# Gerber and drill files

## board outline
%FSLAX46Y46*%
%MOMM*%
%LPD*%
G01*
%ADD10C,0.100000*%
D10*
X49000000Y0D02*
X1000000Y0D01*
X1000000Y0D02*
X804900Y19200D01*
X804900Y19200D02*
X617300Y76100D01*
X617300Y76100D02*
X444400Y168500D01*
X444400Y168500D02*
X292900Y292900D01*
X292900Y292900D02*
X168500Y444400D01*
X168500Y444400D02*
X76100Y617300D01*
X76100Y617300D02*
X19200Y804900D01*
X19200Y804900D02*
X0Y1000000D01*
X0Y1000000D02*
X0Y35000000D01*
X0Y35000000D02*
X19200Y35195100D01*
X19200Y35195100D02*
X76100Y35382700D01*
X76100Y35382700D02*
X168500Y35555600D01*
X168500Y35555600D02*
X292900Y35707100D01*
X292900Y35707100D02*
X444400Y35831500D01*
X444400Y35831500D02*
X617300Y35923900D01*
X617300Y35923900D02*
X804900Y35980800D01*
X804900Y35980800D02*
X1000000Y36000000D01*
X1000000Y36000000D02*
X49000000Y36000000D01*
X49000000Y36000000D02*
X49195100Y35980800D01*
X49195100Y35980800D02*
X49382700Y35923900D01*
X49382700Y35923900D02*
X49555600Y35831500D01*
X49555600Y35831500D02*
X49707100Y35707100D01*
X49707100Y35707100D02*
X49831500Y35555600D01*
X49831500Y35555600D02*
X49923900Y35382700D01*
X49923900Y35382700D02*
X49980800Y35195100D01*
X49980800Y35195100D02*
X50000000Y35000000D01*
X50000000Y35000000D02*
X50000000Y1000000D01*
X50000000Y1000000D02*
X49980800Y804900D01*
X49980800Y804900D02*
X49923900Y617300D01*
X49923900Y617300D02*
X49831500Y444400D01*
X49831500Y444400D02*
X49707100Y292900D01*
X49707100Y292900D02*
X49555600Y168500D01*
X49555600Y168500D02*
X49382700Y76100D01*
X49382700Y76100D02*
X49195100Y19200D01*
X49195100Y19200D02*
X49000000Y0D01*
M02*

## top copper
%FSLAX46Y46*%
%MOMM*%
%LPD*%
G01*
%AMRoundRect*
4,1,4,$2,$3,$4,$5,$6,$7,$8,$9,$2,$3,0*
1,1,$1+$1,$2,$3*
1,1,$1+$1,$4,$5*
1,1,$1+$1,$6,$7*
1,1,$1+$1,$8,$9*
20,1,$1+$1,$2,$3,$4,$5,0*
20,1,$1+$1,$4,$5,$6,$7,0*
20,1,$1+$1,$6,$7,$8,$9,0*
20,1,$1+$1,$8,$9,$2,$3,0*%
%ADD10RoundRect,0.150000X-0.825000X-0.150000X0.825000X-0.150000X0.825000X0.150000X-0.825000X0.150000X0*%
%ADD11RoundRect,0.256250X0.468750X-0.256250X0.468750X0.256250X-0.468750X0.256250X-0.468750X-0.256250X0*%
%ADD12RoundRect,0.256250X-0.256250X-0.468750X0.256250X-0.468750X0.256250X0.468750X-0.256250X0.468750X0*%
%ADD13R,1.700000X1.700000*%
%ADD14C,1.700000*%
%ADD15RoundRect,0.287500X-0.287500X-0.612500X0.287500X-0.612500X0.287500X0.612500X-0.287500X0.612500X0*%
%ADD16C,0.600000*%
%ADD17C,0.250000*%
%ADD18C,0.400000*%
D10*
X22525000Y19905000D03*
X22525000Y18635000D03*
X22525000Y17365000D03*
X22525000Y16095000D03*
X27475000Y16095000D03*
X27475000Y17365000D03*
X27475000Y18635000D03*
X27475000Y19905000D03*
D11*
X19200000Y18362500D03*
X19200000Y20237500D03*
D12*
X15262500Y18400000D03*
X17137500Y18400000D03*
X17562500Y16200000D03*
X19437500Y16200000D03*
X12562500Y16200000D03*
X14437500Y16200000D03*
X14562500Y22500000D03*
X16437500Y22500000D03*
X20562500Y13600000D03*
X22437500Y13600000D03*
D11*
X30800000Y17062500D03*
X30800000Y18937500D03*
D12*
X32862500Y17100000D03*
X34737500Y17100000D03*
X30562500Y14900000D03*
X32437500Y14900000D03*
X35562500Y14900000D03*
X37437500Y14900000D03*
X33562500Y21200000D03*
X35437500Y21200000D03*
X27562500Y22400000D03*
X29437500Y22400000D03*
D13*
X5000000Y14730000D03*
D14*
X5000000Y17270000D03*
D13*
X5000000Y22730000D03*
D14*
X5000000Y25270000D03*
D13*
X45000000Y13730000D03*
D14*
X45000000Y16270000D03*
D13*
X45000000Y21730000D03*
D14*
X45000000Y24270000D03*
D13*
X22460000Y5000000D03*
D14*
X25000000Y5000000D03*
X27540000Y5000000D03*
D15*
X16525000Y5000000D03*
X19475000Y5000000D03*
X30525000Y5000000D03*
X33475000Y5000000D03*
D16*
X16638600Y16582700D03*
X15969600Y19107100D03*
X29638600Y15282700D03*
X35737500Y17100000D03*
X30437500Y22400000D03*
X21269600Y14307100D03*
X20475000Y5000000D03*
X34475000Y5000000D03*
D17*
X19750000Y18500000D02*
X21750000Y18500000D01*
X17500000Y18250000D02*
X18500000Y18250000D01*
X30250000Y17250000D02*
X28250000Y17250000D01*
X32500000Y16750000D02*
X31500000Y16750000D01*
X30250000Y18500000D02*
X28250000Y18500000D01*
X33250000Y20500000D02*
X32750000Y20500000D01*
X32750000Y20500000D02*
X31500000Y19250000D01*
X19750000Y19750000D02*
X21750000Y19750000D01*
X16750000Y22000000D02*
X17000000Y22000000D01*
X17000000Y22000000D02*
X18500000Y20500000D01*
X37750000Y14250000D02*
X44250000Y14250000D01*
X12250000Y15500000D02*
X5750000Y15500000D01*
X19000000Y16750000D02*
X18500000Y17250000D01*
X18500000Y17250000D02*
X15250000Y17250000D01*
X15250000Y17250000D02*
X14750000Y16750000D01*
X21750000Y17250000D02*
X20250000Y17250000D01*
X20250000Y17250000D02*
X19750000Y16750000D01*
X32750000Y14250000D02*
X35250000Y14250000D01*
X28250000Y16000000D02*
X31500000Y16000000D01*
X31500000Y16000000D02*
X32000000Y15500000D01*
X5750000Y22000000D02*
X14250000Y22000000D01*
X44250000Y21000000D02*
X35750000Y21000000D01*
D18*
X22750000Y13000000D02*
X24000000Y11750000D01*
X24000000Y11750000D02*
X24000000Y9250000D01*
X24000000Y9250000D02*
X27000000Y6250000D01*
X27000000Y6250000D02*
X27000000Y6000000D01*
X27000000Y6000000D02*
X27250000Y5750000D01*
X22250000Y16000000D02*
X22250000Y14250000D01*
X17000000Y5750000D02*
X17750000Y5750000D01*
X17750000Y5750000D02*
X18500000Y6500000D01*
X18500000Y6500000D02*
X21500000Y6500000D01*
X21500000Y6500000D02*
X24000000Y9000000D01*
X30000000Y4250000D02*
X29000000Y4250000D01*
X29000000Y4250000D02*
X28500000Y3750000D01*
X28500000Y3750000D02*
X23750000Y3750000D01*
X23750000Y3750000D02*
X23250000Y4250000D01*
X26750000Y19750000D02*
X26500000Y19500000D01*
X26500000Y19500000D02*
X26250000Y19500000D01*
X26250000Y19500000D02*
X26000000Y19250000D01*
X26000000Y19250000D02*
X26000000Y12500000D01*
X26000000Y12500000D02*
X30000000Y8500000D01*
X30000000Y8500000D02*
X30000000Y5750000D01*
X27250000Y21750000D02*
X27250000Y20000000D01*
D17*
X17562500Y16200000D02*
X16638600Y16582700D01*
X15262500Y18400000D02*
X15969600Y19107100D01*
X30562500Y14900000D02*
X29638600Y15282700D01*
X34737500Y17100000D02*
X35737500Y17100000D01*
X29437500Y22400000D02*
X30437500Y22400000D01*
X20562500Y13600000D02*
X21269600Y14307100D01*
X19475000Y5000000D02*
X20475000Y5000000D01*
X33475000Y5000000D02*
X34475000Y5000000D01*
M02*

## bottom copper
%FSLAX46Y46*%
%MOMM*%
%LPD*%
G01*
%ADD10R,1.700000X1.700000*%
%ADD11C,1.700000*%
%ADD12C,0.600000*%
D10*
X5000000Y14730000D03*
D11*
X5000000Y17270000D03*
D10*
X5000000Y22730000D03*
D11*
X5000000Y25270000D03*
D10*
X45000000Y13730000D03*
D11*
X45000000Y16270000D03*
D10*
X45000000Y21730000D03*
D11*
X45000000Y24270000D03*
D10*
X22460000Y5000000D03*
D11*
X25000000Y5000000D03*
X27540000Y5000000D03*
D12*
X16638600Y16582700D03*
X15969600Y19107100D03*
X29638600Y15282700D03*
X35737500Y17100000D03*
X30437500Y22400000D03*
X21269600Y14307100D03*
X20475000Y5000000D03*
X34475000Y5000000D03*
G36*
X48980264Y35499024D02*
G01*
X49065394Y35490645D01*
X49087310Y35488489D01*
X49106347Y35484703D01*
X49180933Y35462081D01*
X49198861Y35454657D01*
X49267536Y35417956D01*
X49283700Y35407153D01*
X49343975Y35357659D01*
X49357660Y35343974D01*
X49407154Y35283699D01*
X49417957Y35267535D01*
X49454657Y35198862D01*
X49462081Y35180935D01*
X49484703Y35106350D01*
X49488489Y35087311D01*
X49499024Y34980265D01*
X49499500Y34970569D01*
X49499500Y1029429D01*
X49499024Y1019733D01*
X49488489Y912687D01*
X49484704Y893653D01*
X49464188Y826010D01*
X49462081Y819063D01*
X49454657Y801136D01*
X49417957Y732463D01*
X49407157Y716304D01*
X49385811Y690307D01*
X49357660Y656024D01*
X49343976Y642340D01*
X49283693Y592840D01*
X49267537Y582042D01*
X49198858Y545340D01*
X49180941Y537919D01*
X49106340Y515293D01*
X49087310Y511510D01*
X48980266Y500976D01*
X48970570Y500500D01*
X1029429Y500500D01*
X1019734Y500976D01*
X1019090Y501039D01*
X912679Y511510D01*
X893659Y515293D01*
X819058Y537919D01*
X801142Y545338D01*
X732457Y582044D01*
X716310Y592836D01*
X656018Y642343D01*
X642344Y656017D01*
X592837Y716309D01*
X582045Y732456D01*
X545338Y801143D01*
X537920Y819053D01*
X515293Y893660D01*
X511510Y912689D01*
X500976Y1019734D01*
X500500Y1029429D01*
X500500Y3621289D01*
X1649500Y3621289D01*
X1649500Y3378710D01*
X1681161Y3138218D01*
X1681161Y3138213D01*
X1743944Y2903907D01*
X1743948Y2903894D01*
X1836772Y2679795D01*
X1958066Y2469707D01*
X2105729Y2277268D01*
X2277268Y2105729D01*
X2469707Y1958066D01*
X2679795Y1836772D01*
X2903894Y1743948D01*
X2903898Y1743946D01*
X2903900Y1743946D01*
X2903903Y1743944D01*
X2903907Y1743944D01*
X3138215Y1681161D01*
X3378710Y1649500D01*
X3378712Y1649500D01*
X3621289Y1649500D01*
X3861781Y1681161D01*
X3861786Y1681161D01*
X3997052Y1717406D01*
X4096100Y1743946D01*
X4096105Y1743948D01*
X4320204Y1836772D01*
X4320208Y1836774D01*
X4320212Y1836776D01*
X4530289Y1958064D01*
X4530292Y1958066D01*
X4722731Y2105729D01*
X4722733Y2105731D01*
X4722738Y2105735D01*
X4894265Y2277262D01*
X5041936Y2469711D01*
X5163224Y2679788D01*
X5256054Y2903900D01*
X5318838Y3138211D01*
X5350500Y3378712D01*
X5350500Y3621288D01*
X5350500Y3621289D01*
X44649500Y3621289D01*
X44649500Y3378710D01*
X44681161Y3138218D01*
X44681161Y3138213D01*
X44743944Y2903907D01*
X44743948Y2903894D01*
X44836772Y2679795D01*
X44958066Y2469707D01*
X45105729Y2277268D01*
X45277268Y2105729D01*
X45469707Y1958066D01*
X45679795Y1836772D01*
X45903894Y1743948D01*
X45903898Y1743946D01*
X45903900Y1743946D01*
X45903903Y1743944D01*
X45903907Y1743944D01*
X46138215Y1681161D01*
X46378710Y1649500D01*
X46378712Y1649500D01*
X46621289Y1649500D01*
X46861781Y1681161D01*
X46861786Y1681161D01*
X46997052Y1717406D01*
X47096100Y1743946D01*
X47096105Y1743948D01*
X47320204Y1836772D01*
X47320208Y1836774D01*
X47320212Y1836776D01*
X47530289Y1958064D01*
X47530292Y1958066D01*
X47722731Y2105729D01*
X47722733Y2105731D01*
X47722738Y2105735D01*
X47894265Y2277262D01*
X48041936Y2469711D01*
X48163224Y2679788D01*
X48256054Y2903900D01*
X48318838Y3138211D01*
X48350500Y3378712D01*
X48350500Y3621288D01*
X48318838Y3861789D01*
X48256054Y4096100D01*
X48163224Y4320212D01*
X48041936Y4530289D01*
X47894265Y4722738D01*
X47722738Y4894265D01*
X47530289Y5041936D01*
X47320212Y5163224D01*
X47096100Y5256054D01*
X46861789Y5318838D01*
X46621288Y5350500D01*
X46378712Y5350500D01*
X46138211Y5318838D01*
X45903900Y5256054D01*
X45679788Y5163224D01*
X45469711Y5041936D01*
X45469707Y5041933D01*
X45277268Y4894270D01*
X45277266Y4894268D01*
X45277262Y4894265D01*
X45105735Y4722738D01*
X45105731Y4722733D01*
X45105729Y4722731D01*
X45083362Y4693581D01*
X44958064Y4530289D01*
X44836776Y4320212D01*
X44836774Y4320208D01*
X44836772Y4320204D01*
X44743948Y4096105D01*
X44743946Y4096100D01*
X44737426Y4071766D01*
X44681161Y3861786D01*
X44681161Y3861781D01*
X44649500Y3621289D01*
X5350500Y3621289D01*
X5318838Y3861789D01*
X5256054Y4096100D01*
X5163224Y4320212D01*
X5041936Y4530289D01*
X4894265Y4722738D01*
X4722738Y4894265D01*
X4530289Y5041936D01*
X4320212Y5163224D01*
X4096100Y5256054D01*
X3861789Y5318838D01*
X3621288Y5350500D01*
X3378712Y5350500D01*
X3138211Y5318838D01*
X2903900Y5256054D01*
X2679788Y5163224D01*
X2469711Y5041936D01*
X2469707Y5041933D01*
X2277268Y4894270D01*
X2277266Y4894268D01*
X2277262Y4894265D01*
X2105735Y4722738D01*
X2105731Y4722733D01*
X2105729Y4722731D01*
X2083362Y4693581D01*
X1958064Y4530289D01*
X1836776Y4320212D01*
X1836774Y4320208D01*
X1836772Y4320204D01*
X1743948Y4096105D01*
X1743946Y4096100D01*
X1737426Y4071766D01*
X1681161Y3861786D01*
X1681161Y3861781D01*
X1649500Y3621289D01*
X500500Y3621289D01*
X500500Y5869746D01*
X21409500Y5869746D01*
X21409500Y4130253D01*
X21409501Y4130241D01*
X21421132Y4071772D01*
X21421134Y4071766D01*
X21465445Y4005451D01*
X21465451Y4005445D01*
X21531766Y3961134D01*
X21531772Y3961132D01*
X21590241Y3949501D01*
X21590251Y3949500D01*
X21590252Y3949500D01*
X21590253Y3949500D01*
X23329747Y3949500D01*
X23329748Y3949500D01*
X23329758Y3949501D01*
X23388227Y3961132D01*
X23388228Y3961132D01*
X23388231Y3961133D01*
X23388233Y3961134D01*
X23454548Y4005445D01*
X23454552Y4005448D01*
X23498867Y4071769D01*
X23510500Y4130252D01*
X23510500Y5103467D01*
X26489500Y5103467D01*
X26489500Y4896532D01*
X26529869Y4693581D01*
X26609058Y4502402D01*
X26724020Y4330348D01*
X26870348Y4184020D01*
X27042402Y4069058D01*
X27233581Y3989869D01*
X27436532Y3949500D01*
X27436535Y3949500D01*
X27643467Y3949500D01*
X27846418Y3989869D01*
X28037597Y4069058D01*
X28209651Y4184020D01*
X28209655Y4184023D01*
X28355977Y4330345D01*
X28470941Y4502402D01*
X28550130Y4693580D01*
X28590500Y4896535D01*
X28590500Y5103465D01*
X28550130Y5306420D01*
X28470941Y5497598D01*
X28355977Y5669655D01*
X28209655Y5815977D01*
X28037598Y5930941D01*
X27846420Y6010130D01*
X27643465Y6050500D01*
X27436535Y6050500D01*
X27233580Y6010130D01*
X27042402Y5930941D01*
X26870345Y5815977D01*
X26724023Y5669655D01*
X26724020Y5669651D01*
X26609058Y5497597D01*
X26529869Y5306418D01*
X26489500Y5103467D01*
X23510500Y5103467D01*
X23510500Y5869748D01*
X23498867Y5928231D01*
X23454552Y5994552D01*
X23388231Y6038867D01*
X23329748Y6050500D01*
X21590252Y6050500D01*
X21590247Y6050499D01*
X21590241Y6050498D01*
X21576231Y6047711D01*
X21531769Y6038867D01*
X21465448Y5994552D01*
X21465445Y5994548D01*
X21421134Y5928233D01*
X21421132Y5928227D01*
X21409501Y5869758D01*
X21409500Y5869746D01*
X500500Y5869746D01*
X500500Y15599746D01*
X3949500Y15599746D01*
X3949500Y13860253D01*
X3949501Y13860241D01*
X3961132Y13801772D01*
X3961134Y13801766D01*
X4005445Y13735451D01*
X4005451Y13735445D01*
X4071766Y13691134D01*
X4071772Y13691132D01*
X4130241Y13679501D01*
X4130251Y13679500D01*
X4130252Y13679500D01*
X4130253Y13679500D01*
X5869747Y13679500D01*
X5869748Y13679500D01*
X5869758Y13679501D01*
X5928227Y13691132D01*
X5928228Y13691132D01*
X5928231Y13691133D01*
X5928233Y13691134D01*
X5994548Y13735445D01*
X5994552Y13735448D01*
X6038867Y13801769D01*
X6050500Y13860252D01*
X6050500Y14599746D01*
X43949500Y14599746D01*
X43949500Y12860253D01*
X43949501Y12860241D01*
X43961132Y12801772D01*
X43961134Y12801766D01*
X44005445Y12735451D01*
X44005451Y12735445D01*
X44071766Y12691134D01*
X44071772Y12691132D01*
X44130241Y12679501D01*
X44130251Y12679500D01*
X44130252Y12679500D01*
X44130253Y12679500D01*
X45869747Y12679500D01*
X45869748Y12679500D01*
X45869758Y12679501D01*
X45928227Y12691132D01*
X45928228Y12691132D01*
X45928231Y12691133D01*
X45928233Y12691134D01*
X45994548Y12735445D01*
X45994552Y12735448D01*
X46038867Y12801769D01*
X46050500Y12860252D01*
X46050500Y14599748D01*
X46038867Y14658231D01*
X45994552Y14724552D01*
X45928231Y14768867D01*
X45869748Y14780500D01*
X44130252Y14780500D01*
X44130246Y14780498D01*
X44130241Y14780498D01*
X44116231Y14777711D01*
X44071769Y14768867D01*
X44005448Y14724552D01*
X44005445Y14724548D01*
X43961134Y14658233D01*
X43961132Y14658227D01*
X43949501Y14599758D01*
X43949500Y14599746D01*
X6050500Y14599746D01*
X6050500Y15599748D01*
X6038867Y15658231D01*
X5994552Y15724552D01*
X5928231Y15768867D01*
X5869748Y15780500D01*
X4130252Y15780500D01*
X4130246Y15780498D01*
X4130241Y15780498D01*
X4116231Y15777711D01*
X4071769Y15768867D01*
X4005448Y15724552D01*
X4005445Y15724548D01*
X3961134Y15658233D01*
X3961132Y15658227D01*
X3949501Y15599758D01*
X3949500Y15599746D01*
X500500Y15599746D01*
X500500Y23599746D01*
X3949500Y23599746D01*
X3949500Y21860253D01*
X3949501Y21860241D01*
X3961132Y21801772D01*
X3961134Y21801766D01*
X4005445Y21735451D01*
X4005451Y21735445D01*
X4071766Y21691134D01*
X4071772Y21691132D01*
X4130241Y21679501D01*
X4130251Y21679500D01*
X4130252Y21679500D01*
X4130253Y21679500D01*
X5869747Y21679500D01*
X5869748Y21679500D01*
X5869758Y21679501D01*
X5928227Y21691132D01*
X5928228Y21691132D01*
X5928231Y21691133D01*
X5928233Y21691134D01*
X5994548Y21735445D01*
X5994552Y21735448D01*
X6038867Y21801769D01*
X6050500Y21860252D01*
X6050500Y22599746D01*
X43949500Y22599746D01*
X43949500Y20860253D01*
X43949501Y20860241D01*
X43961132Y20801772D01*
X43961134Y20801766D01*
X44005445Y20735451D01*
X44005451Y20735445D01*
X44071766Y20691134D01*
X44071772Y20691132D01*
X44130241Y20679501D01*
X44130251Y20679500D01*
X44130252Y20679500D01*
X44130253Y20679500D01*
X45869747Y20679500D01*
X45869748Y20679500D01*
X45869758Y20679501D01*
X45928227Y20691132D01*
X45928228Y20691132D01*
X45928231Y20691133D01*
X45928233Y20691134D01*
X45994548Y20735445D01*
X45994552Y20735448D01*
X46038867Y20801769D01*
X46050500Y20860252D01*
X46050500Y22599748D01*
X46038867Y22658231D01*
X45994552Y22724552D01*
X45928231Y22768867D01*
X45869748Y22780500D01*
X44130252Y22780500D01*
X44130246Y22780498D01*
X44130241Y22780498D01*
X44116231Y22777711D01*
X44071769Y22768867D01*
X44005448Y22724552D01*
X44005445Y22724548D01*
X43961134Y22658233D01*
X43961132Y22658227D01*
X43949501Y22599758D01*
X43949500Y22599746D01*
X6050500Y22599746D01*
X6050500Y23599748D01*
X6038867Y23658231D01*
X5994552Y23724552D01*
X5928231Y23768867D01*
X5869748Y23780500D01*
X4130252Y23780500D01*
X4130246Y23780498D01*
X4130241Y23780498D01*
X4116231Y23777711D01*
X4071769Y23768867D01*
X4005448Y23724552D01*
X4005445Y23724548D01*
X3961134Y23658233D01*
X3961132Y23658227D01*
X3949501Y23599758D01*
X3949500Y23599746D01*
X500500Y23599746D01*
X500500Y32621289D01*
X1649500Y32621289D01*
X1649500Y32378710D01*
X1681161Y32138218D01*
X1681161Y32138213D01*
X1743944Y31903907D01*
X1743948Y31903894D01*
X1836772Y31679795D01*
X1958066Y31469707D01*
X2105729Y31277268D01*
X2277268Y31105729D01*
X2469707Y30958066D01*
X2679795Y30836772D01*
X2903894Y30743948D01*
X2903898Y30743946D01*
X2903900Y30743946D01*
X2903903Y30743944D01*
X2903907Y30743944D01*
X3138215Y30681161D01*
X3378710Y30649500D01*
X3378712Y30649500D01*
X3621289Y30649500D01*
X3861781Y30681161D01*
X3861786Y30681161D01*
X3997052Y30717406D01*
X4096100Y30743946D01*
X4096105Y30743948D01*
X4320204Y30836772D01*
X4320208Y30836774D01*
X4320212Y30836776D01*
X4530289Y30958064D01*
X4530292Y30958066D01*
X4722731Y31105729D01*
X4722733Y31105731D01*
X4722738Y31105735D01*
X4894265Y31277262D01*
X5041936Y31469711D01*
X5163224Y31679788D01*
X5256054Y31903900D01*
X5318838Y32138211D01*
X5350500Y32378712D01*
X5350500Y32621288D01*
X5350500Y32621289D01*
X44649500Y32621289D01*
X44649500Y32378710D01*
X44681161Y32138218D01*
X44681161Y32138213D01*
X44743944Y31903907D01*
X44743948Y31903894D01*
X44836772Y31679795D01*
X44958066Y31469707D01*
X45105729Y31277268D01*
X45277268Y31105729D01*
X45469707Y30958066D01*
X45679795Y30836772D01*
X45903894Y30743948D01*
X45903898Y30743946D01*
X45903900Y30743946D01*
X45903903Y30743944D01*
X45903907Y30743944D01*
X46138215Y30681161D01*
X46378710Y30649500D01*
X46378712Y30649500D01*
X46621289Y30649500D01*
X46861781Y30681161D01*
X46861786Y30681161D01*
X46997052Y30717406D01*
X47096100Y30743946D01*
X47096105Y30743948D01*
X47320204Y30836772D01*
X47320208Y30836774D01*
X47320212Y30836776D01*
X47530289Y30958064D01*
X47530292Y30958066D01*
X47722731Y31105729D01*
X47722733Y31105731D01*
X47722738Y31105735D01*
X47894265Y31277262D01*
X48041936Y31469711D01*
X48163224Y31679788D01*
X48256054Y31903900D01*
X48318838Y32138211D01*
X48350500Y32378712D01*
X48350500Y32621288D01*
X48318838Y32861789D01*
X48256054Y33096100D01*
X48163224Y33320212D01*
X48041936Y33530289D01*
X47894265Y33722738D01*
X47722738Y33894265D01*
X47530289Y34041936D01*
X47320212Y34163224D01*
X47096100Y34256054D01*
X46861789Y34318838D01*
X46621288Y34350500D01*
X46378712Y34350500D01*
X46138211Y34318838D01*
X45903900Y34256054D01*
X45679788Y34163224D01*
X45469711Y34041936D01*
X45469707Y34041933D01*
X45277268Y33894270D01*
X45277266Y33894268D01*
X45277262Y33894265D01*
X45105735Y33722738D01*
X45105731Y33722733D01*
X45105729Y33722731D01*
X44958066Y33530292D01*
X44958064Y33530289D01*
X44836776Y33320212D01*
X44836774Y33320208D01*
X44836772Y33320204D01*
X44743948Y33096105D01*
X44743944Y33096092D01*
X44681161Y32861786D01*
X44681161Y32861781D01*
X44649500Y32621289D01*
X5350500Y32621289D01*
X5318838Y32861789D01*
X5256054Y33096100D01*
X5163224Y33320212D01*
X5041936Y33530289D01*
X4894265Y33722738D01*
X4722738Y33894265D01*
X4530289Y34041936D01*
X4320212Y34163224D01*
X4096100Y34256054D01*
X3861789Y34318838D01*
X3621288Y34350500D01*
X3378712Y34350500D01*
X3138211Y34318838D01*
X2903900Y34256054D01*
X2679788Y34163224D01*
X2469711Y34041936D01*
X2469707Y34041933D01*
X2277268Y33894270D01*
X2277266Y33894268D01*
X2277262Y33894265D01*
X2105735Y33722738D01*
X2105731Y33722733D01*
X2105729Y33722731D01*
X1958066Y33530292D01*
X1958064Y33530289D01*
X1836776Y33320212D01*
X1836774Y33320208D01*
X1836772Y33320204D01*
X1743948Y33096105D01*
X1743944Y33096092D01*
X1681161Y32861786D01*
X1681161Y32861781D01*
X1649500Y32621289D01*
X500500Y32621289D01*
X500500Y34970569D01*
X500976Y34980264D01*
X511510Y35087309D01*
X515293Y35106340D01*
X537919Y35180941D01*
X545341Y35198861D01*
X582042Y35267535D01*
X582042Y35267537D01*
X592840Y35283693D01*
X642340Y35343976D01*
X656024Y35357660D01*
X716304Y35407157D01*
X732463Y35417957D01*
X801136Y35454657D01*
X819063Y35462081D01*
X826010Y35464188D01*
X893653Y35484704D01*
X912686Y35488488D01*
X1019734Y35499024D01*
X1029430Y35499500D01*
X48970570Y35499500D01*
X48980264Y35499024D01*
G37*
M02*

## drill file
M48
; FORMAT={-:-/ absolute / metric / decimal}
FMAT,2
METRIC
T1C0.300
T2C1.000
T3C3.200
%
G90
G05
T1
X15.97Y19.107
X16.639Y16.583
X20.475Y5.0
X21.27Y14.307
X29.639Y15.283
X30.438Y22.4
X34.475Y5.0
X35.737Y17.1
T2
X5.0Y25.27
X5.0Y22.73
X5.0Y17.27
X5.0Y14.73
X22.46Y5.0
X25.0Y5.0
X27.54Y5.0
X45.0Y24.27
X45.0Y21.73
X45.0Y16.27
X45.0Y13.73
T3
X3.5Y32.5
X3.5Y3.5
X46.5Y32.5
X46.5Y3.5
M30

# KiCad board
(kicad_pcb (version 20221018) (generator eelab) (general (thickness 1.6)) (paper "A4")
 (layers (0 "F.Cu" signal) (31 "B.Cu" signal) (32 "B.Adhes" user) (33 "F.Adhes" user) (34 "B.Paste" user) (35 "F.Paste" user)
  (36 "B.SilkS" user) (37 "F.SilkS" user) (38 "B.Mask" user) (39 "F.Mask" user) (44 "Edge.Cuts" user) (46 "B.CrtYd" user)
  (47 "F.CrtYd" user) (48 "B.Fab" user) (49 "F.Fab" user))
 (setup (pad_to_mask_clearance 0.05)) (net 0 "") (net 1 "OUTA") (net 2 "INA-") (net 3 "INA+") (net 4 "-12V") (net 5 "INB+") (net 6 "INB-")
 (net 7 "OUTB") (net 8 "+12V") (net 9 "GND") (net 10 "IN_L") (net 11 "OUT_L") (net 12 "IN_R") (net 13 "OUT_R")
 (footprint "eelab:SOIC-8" (layer "F.Cu") (at 25.0000 -18.0000 0)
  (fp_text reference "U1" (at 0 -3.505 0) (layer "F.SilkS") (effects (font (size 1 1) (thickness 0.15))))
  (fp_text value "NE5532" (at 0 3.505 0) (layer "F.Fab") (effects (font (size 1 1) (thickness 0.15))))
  (pad "1" smd roundrect (at -2.4750 -1.9050 0) (size 1.9500 0.6000) (layers "F.Cu" "F.Paste" "F.Mask") (roundrect_rratio 0.25)
   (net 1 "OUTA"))
  (pad "2" smd roundrect (at -2.4750 -0.6350 0) (size 1.9500 0.6000) (layers "F.Cu" "F.Paste" "F.Mask") (roundrect_rratio 0.25)
   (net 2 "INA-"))
  (pad "3" smd roundrect (at -2.4750 0.6350 0) (size 1.9500 0.6000) (layers "F.Cu" "F.Paste" "F.Mask") (roundrect_rratio 0.25)
   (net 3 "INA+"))
  (pad "4" smd roundrect (at -2.4750 1.9050 0) (size 1.9500 0.6000) (layers "F.Cu" "F.Paste" "F.Mask") (roundrect_rratio 0.25)
   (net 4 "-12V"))
  (pad "5" smd roundrect (at 2.4750 1.9050 0) (size 1.9500 0.6000) (layers "F.Cu" "F.Paste" "F.Mask") (roundrect_rratio 0.25) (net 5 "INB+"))
  (pad "6" smd roundrect (at 2.4750 0.6350 0) (size 1.9500 0.6000) (layers "F.Cu" "F.Paste" "F.Mask") (roundrect_rratio 0.25) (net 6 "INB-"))
  (pad "7" smd roundrect (at 2.4750 -0.6350 0) (size 1.9500 0.6000) (layers "F.Cu" "F.Paste" "F.Mask") (roundrect_rratio 0.25)
   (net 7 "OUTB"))
  (pad "8" smd roundrect (at 2.4750 -1.9050 0) (size 1.9500 0.6000) (layers "F.Cu" "F.Paste" "F.Mask") (roundrect_rratio 0.25)
   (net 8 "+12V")))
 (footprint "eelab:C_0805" (layer "F.Cu") (at 19.2000 -19.3000 90)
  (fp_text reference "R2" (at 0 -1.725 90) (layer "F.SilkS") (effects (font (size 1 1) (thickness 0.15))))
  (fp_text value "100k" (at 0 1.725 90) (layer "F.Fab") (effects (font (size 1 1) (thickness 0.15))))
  (pad "1" smd roundrect (at -0.9375 0.0000 90) (size 1.0250 1.4500) (layers "F.Cu" "F.Paste" "F.Mask") (roundrect_rratio 0.25)
   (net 2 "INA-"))
  (pad "2" smd roundrect (at 0.9375 0.0000 90) (size 1.0250 1.4500) (layers "F.Cu" "F.Paste" "F.Mask") (roundrect_rratio 0.25)
   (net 1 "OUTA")))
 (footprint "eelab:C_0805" (layer "F.Cu") (at 16.2000 -18.4000 0)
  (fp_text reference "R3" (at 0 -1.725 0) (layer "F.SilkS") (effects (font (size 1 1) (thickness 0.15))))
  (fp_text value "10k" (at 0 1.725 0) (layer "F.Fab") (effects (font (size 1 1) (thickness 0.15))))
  (pad "1" smd roundrect (at -0.9375 0.0000 0) (size 1.0250 1.4500) (layers "F.Cu" "F.Paste" "F.Mask") (roundrect_rratio 0.25) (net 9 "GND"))
  (pad "2" smd roundrect (at 0.9375 0.0000 0) (size 1.0250 1.4500) (layers "F.Cu" "F.Paste" "F.Mask") (roundrect_rratio 0.25) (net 2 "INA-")))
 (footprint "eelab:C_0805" (layer "F.Cu") (at 18.5000 -16.2000 0)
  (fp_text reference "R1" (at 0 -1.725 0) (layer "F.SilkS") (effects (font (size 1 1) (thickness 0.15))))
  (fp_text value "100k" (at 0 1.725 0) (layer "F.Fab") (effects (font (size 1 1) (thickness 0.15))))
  (pad "1" smd roundrect (at -0.9375 0.0000 0) (size 1.0250 1.4500) (layers "F.Cu" "F.Paste" "F.Mask") (roundrect_rratio 0.25) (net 9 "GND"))
  (pad "2" smd roundrect (at 0.9375 0.0000 0) (size 1.0250 1.4500) (layers "F.Cu" "F.Paste" "F.Mask") (roundrect_rratio 0.25) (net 3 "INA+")))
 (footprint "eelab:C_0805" (layer "F.Cu") (at 13.5000 -16.2000 0)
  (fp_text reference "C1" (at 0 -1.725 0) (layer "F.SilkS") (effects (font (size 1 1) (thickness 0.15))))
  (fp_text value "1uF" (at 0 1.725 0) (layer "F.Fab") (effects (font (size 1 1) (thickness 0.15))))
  (pad "1" smd roundrect (at -0.9375 0.0000 0) (size 1.0250 1.4500) (layers "F.Cu" "F.Paste" "F.Mask") (roundrect_rratio 0.25)
   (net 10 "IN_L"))
  (pad "2" smd roundrect (at 0.9375 0.0000 0) (size 1.0250 1.4500) (layers "F.Cu" "F.Paste" "F.Mask") (roundrect_rratio 0.25) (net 3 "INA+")))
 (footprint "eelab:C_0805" (layer "F.Cu") (at 15.5000 -22.5000 0)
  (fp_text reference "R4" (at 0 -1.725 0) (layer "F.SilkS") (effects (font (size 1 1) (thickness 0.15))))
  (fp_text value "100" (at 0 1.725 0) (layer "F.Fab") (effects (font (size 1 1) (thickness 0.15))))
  (pad "1" smd roundrect (at -0.9375 0.0000 0) (size 1.0250 1.4500) (layers "F.Cu" "F.Paste" "F.Mask") (roundrect_rratio 0.25)
   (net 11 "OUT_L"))
  (pad "2" smd roundrect (at 0.9375 0.0000 0) (size 1.0250 1.4500) (layers "F.Cu" "F.Paste" "F.Mask") (roundrect_rratio 0.25) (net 1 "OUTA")))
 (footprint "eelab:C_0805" (layer "F.Cu") (at 21.5000 -13.6000 0)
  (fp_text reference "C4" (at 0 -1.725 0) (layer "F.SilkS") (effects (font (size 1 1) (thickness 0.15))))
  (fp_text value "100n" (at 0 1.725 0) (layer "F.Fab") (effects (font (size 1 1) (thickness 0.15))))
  (pad "1" smd roundrect (at -0.9375 0.0000 0) (size 1.0250 1.4500) (layers "F.Cu" "F.Paste" "F.Mask") (roundrect_rratio 0.25) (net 9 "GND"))
  (pad "2" smd roundrect (at 0.9375 0.0000 0) (size 1.0250 1.4500) (layers "F.Cu" "F.Paste" "F.Mask") (roundrect_rratio 0.25) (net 4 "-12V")))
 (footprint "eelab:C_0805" (layer "F.Cu") (at 30.8000 -18.0000 90)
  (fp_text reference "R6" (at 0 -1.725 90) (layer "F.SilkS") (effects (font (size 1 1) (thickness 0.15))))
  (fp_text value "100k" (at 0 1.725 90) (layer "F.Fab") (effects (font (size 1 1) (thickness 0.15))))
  (pad "1" smd roundrect (at -0.9375 0.0000 90) (size 1.0250 1.4500) (layers "F.Cu" "F.Paste" "F.Mask") (roundrect_rratio 0.25)
   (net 6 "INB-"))
  (pad "2" smd roundrect (at 0.9375 0.0000 90) (size 1.0250 1.4500) (layers "F.Cu" "F.Paste" "F.Mask") (roundrect_rratio 0.25)
   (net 7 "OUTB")))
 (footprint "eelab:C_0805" (layer "F.Cu") (at 33.8000 -17.1000 0)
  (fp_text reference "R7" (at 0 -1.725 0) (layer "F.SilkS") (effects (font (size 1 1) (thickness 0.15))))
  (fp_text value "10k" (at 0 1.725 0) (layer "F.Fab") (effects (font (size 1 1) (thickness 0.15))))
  (pad "1" smd roundrect (at -0.9375 0.0000 0) (size 1.0250 1.4500) (layers "F.Cu" "F.Paste" "F.Mask") (roundrect_rratio 0.25)
   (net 6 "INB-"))
  (pad "2" smd roundrect (at 0.9375 0.0000 0) (size 1.0250 1.4500) (layers "F.Cu" "F.Paste" "F.Mask") (roundrect_rratio 0.25) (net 9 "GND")))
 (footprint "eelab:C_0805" (layer "F.Cu") (at 31.5000 -14.9000 0)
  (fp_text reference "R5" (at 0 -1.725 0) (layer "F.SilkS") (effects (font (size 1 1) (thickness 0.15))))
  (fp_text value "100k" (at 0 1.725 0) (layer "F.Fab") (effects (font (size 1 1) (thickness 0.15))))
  (pad "1" smd roundrect (at -0.9375 0.0000 0) (size 1.0250 1.4500) (layers "F.Cu" "F.Paste" "F.Mask") (roundrect_rratio 0.25) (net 9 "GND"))
  (pad "2" smd roundrect (at 0.9375 0.0000 0) (size 1.0250 1.4500) (layers "F.Cu" "F.Paste" "F.Mask") (roundrect_rratio 0.25) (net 5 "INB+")))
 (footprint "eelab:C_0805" (layer "F.Cu") (at 36.5000 -14.9000 0)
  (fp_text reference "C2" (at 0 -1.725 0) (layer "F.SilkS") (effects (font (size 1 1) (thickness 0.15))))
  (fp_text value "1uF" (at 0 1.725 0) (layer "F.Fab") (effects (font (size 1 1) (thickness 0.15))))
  (pad "1" smd roundrect (at -0.9375 0.0000 0) (size 1.0250 1.4500) (layers "F.Cu" "F.Paste" "F.Mask") (roundrect_rratio 0.25)
   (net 5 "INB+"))
  (pad "2" smd roundrect (at 0.9375 0.0000 0) (size 1.0250 1.4500) (layers "F.Cu" "F.Paste" "F.Mask") (roundrect_rratio 0.25)
   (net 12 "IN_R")))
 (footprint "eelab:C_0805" (layer "F.Cu") (at 34.5000 -21.2000 0)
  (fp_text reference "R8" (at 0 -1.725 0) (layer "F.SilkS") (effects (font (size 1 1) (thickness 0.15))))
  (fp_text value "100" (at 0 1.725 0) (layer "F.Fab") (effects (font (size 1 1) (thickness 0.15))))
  (pad "1" smd roundrect (at -0.9375 0.0000 0) (size 1.0250 1.4500) (layers "F.Cu" "F.Paste" "F.Mask") (roundrect_rratio 0.25)
   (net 7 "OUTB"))
  (pad "2" smd roundrect (at 0.9375 0.0000 0) (size 1.0250 1.4500) (layers "F.Cu" "F.Paste" "F.Mask") (roundrect_rratio 0.25)
   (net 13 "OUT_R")))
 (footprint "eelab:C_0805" (layer "F.Cu") (at 28.5000 -22.4000 0)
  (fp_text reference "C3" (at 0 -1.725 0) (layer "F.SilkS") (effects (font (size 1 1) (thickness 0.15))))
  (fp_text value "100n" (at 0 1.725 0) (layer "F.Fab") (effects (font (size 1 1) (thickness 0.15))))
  (pad "1" smd roundrect (at -0.9375 0.0000 0) (size 1.0250 1.4500) (layers "F.Cu" "F.Paste" "F.Mask") (roundrect_rratio 0.25)
   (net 8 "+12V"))
  (pad "2" smd roundrect (at 0.9375 0.0000 0) (size 1.0250 1.4500) (layers "F.Cu" "F.Paste" "F.Mask") (roundrect_rratio 0.25) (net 9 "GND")))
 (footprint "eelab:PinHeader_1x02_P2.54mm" (layer "F.Cu") (at 5.0000 -16.0000 90)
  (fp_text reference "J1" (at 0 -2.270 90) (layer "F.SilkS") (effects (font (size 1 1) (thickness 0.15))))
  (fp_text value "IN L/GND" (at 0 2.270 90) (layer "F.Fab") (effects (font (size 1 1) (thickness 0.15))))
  (pad "1" thru_hole rect (at -1.2700 -0.0000 90) (size 1.7000 1.7000) (drill 1.0) (layers "*.Cu" "*.Mask") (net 10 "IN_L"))
  (pad "2" thru_hole circle (at 1.2700 -0.0000 90) (size 1.7000 1.7000) (drill 1.0) (layers "*.Cu" "*.Mask") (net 9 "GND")))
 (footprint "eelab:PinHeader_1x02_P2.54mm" (layer "F.Cu") (at 5.0000 -24.0000 90)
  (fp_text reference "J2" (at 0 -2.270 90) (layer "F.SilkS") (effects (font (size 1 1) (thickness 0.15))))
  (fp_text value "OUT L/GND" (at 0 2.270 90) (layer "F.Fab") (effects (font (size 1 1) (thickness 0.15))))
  (pad "1" thru_hole rect (at -1.2700 -0.0000 90) (size 1.7000 1.7000) (drill 1.0) (layers "*.Cu" "*.Mask") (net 11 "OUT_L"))
  (pad "2" thru_hole circle (at 1.2700 -0.0000 90) (size 1.7000 1.7000) (drill 1.0) (layers "*.Cu" "*.Mask") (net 9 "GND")))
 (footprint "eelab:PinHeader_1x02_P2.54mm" (layer "F.Cu") (at 45.0000 -15.0000 90)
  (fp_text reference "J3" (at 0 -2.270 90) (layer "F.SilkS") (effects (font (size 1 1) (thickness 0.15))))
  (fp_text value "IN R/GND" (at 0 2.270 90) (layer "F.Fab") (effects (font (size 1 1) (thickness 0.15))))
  (pad "1" thru_hole rect (at -1.2700 -0.0000 90) (size 1.7000 1.7000) (drill 1.0) (layers "*.Cu" "*.Mask") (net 12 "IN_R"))
  (pad "2" thru_hole circle (at 1.2700 -0.0000 90) (size 1.7000 1.7000) (drill 1.0) (layers "*.Cu" "*.Mask") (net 9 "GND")))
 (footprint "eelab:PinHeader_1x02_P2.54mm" (layer "F.Cu") (at 45.0000 -23.0000 90)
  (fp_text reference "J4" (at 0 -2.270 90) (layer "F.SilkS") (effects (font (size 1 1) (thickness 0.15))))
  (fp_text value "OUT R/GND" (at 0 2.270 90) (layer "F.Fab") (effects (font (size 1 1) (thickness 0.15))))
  (pad "1" thru_hole rect (at -1.2700 -0.0000 90) (size 1.7000 1.7000) (drill 1.0) (layers "*.Cu" "*.Mask") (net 13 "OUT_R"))
  (pad "2" thru_hole circle (at 1.2700 -0.0000 90) (size 1.7000 1.7000) (drill 1.0) (layers "*.Cu" "*.Mask") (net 9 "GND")))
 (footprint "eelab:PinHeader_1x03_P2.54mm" (layer "F.Cu") (at 25.0000 -5.0000 0)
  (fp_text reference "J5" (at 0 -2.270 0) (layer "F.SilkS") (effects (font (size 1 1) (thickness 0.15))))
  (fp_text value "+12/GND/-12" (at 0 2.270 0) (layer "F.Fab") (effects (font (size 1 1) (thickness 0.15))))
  (pad "1" thru_hole rect (at -2.5400 -0.0000 0) (size 1.7000 1.7000) (drill 1.0) (layers "*.Cu" "*.Mask") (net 8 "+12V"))
  (pad "2" thru_hole circle (at 0.0000 -0.0000 0) (size 1.7000 1.7000) (drill 1.0) (layers "*.Cu" "*.Mask") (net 9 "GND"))
  (pad "3" thru_hole circle (at 2.5400 -0.0000 0) (size 1.7000 1.7000) (drill 1.0) (layers "*.Cu" "*.Mask") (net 4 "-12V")))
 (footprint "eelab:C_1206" (layer "F.Cu") (at 18.0000 -5.0000 0)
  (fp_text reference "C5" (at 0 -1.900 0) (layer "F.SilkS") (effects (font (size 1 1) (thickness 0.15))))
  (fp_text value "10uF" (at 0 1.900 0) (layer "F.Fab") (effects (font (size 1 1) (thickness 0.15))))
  (pad "1" smd roundrect (at -1.4750 0.0000 0) (size 1.1500 1.8000) (layers "F.Cu" "F.Paste" "F.Mask") (roundrect_rratio 0.25)
   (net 4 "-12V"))
  (pad "2" smd roundrect (at 1.4750 0.0000 0) (size 1.1500 1.8000) (layers "F.Cu" "F.Paste" "F.Mask") (roundrect_rratio 0.25) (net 9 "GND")))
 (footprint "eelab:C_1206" (layer "F.Cu") (at 32.0000 -5.0000 0)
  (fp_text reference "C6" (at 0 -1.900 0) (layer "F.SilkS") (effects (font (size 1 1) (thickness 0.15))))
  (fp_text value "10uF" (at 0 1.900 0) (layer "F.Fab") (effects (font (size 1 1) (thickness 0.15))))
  (pad "1" smd roundrect (at -1.4750 0.0000 0) (size 1.1500 1.8000) (layers "F.Cu" "F.Paste" "F.Mask") (roundrect_rratio 0.25)
   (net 8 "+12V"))
  (pad "2" smd roundrect (at 1.4750 0.0000 0) (size 1.1500 1.8000) (layers "F.Cu" "F.Paste" "F.Mask") (roundrect_rratio 0.25) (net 9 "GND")))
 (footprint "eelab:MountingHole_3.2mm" (layer "F.Cu") (at 3.5000 -3.5000 0)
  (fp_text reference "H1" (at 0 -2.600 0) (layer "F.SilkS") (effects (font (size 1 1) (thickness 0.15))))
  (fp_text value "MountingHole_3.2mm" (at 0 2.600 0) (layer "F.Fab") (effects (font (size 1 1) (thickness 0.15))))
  (pad "" np_thru_hole circle (at 0.0000 0.0000 0) (size 3.2000 3.2000) (drill 3.2) (layers "*.Cu" "*.Mask")))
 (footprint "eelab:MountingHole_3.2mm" (layer "F.Cu") (at 46.5000 -3.5000 0)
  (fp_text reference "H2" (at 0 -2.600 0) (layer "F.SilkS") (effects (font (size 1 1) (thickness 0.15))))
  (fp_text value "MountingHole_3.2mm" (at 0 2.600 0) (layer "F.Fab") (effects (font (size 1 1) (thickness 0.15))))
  (pad "" np_thru_hole circle (at 0.0000 0.0000 0) (size 3.2000 3.2000) (drill 3.2) (layers "*.Cu" "*.Mask")))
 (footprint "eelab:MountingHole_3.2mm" (layer "F.Cu") (at 3.5000 -32.5000 0)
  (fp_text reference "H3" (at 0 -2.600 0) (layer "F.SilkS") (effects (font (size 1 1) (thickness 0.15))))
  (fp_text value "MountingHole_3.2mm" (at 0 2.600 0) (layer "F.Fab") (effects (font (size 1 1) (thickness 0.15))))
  (pad "" np_thru_hole circle (at 0.0000 0.0000 0) (size 3.2000 3.2000) (drill 3.2) (layers "*.Cu" "*.Mask")))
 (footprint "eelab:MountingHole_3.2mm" (layer "F.Cu") (at 46.5000 -32.5000 0)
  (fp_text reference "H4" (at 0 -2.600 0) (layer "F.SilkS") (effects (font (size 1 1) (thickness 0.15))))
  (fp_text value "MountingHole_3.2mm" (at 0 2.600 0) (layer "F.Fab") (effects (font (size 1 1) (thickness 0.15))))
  (pad "" np_thru_hole circle (at 0.0000 0.0000 0) (size 3.2000 3.2000) (drill 3.2) (layers "*.Cu" "*.Mask")))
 (gr_line (start 49.0000 -0.0000) (end 1.0000 -0.0000) (stroke (width 0.1) (type solid)) (layer "Edge.Cuts"))
 (gr_line (start 1.0000 -0.0000) (end 0.8049 -0.0192) (stroke (width 0.1) (type solid)) (layer "Edge.Cuts"))
 (gr_line (start 0.8049 -0.0192) (end 0.6173 -0.0761) (stroke (width 0.1) (type solid)) (layer "Edge.Cuts"))
 (gr_line (start 0.6173 -0.0761) (end 0.4444 -0.1685) (stroke (width 0.1) (type solid)) (layer "Edge.Cuts"))
 (gr_line (start 0.4444 -0.1685) (end 0.2929 -0.2929) (stroke (width 0.1) (type solid)) (layer "Edge.Cuts"))
 (gr_line (start 0.2929 -0.2929) (end 0.1685 -0.4444) (stroke (width 0.1) (type solid)) (layer "Edge.Cuts"))
 (gr_line (start 0.1685 -0.4444) (end 0.0761 -0.6173) (stroke (width 0.1) (type solid)) (layer "Edge.Cuts"))
 (gr_line (start 0.0761 -0.6173) (end 0.0192 -0.8049) (stroke (width 0.1) (type solid)) (layer "Edge.Cuts"))
 (gr_line (start 0.0192 -0.8049) (end 0.0000 -1.0000) (stroke (width 0.1) (type solid)) (layer "Edge.Cuts"))
 (gr_line (start 0.0000 -1.0000) (end 0.0000 -35.0000) (stroke (width 0.1) (type solid)) (layer "Edge.Cuts"))
 (gr_line (start 0.0000 -35.0000) (end 0.0192 -35.1951) (stroke (width 0.1) (type solid)) (layer "Edge.Cuts"))
 (gr_line (start 0.0192 -35.1951) (end 0.0761 -35.3827) (stroke (width 0.1) (type solid)) (layer "Edge.Cuts"))
 (gr_line (start 0.0761 -35.3827) (end 0.1685 -35.5556) (stroke (width 0.1) (type solid)) (layer "Edge.Cuts"))
 (gr_line (start 0.1685 -35.5556) (end 0.2929 -35.7071) (stroke (width 0.1) (type solid)) (layer "Edge.Cuts"))
 (gr_line (start 0.2929 -35.7071) (end 0.4444 -35.8315) (stroke (width 0.1) (type solid)) (layer "Edge.Cuts"))
 (gr_line (start 0.4444 -35.8315) (end 0.6173 -35.9239) (stroke (width 0.1) (type solid)) (layer "Edge.Cuts"))
 (gr_line (start 0.6173 -35.9239) (end 0.8049 -35.9808) (stroke (width 0.1) (type solid)) (layer "Edge.Cuts"))
 (gr_line (start 0.8049 -35.9808) (end 1.0000 -36.0000) (stroke (width 0.1) (type solid)) (layer "Edge.Cuts"))
 (gr_line (start 1.0000 -36.0000) (end 49.0000 -36.0000) (stroke (width 0.1) (type solid)) (layer "Edge.Cuts"))
 (gr_line (start 49.0000 -36.0000) (end 49.1951 -35.9808) (stroke (width 0.1) (type solid)) (layer "Edge.Cuts"))
 (gr_line (start 49.1951 -35.9808) (end 49.3827 -35.9239) (stroke (width 0.1) (type solid)) (layer "Edge.Cuts"))
 (gr_line (start 49.3827 -35.9239) (end 49.5556 -35.8315) (stroke (width 0.1) (type solid)) (layer "Edge.Cuts"))
 (gr_line (start 49.5556 -35.8315) (end 49.7071 -35.7071) (stroke (width 0.1) (type solid)) (layer "Edge.Cuts"))
 (gr_line (start 49.7071 -35.7071) (end 49.8315 -35.5556) (stroke (width 0.1) (type solid)) (layer "Edge.Cuts"))
 (gr_line (start 49.8315 -35.5556) (end 49.9239 -35.3827) (stroke (width 0.1) (type solid)) (layer "Edge.Cuts"))
 (gr_line (start 49.9239 -35.3827) (end 49.9808 -35.1951) (stroke (width 0.1) (type solid)) (layer "Edge.Cuts"))
 (gr_line (start 49.9808 -35.1951) (end 50.0000 -35.0000) (stroke (width 0.1) (type solid)) (layer "Edge.Cuts"))
 (gr_line (start 50.0000 -35.0000) (end 50.0000 -1.0000) (stroke (width 0.1) (type solid)) (layer "Edge.Cuts"))
 (gr_line (start 50.0000 -1.0000) (end 49.9808 -0.8049) (stroke (width 0.1) (type solid)) (layer "Edge.Cuts"))
 (gr_line (start 49.9808 -0.8049) (end 49.9239 -0.6173) (stroke (width 0.1) (type solid)) (layer "Edge.Cuts"))
 (gr_line (start 49.9239 -0.6173) (end 49.8315 -0.4444) (stroke (width 0.1) (type solid)) (layer "Edge.Cuts"))
 (gr_line (start 49.8315 -0.4444) (end 49.7071 -0.2929) (stroke (width 0.1) (type solid)) (layer "Edge.Cuts"))
 (gr_line (start 49.7071 -0.2929) (end 49.5556 -0.1685) (stroke (width 0.1) (type solid)) (layer "Edge.Cuts"))
 (gr_line (start 49.5556 -0.1685) (end 49.3827 -0.0761) (stroke (width 0.1) (type solid)) (layer "Edge.Cuts"))
 (gr_line (start 49.3827 -0.0761) (end 49.1951 -0.0192) (stroke (width 0.1) (type solid)) (layer "Edge.Cuts"))
 (gr_line (start 49.1951 -0.0192) (end 49.0000 -0.0000) (stroke (width 0.1) (type solid)) (layer "Edge.Cuts"))
 (segment (start 19.7500 -18.5000) (end 21.7500 -18.5000) (width 0.25) (layer "F.Cu") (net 2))
 (segment (start 17.5000 -18.2500) (end 18.5000 -18.2500) (width 0.25) (layer "F.Cu") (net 2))
 (segment (start 30.2500 -17.2500) (end 28.2500 -17.2500) (width 0.25) (layer "F.Cu") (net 6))
 (segment (start 32.5000 -16.7500) (end 31.5000 -16.7500) (width 0.25) (layer "F.Cu") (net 6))
 (segment (start 30.2500 -18.5000) (end 28.2500 -18.5000) (width 0.25) (layer "F.Cu") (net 7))
 (segment (start 33.2500 -20.5000) (end 32.7500 -20.5000) (width 0.25) (layer "F.Cu") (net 7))
 (segment (start 32.7500 -20.5000) (end 31.5000 -19.2500) (width 0.25) (layer "F.Cu") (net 7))
 (segment (start 19.7500 -19.7500) (end 21.7500 -19.7500) (width 0.25) (layer "F.Cu") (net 1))
 (segment (start 16.7500 -22.0000) (end 17.0000 -22.0000) (width 0.25) (layer "F.Cu") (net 1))
 (segment (start 17.0000 -22.0000) (end 18.5000 -20.5000) (width 0.25) (layer "F.Cu") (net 1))
 (segment (start 37.7500 -14.2500) (end 44.2500 -14.2500) (width 0.25) (layer "F.Cu") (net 12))
 (segment (start 12.2500 -15.5000) (end 5.7500 -15.5000) (width 0.25) (layer "F.Cu") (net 10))
 (segment (start 19.0000 -16.7500) (end 18.5000 -17.2500) (width 0.25) (layer "F.Cu") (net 3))
 (segment (start 18.5000 -17.2500) (end 15.2500 -17.2500) (width 0.25) (layer "F.Cu") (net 3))
 (segment (start 15.2500 -17.2500) (end 14.7500 -16.7500) (width 0.25) (layer "F.Cu") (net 3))
 (segment (start 21.7500 -17.2500) (end 20.2500 -17.2500) (width 0.25) (layer "F.Cu") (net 3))
 (segment (start 20.2500 -17.2500) (end 19.7500 -16.7500) (width 0.25) (layer "F.Cu") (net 3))
 (segment (start 32.7500 -14.2500) (end 35.2500 -14.2500) (width 0.25) (layer "F.Cu") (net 5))
 (segment (start 28.2500 -16.0000) (end 31.5000 -16.0000) (width 0.25) (layer "F.Cu") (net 5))
 (segment (start 31.5000 -16.0000) (end 32.0000 -15.5000) (width 0.25) (layer "F.Cu") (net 5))
 (segment (start 5.7500 -22.0000) (end 14.2500 -22.0000) (width 0.25) (layer "F.Cu") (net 11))
 (segment (start 44.2500 -21.0000) (end 35.7500 -21.0000) (width 0.25) (layer "F.Cu") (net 13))
 (segment (start 22.7500 -13.0000) (end 24.0000 -11.7500) (width 0.4) (layer "F.Cu") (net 4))
 (segment (start 24.0000 -11.7500) (end 24.0000 -9.2500) (width 0.4) (layer "F.Cu") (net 4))
 (segment (start 24.0000 -9.2500) (end 27.0000 -6.2500) (width 0.4) (layer "F.Cu") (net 4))
 (segment (start 27.0000 -6.2500) (end 27.0000 -6.0000) (width 0.4) (layer "F.Cu") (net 4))
 (segment (start 27.0000 -6.0000) (end 27.2500 -5.7500) (width 0.4) (layer "F.Cu") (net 4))
 (segment (start 22.2500 -16.0000) (end 22.2500 -14.2500) (width 0.4) (layer "F.Cu") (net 4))
 (segment (start 17.0000 -5.7500) (end 17.7500 -5.7500) (width 0.4) (layer "F.Cu") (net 4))
 (segment (start 17.7500 -5.7500) (end 18.5000 -6.5000) (width 0.4) (layer "F.Cu") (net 4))
 (segment (start 18.5000 -6.5000) (end 21.5000 -6.5000) (width 0.4) (layer "F.Cu") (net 4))
 (segment (start 21.5000 -6.5000) (end 24.0000 -9.0000) (width 0.4) (layer "F.Cu") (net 4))
 (segment (start 30.0000 -4.2500) (end 29.0000 -4.2500) (width 0.4) (layer "F.Cu") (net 8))
 (segment (start 29.0000 -4.2500) (end 28.5000 -3.7500) (width 0.4) (layer "F.Cu") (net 8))
 (segment (start 28.5000 -3.7500) (end 23.7500 -3.7500) (width 0.4) (layer "F.Cu") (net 8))
 (segment (start 23.7500 -3.7500) (end 23.2500 -4.2500) (width 0.4) (layer "F.Cu") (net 8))
 (segment (start 26.7500 -19.7500) (end 26.5000 -19.5000) (width 0.4) (layer "F.Cu") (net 8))
 (segment (start 26.5000 -19.5000) (end 26.2500 -19.5000) (width 0.4) (layer "F.Cu") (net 8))
 (segment (start 26.2500 -19.5000) (end 26.0000 -19.2500) (width 0.4) (layer "F.Cu") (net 8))
 (segment (start 26.0000 -19.2500) (end 26.0000 -12.5000) (width 0.4) (layer "F.Cu") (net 8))
 (segment (start 26.0000 -12.5000) (end 30.0000 -8.5000) (width 0.4) (layer "F.Cu") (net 8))
 (segment (start 30.0000 -8.5000) (end 30.0000 -5.7500) (width 0.4) (layer "F.Cu") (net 8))
 (segment (start 27.2500 -21.7500) (end 27.2500 -20.0000) (width 0.4) (layer "F.Cu") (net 8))
 (segment (start 17.5625 -16.2000) (end 16.6386 -16.5827) (width 0.25) (layer "F.Cu") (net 9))
 (segment (start 15.2625 -18.4000) (end 15.9696 -19.1071) (width 0.25) (layer "F.Cu") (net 9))
 (segment (start 30.5625 -14.9000) (end 29.6386 -15.2827) (width 0.25) (layer "F.Cu") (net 9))
 (segment (start 34.7375 -17.1000) (end 35.7375 -17.1000) (width 0.25) (layer "F.Cu") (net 9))
 (segment (start 29.4375 -22.4000) (end 30.4375 -22.4000) (width 0.25) (layer "F.Cu") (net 9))
 (segment (start 20.5625 -13.6000) (end 21.2696 -14.3071) (width 0.25) (layer "F.Cu") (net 9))
 (segment (start 19.4750 -5.0000) (end 20.4750 -5.0000) (width 0.25) (layer "F.Cu") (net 9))
 (segment (start 33.4750 -5.0000) (end 34.4750 -5.0000) (width 0.25) (layer "F.Cu") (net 9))
 (via (at 16.6386 -16.5827) (size 0.6) (drill 0.3) (layers "F.Cu" "B.Cu") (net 9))
 (via (at 15.9696 -19.1071) (size 0.6) (drill 0.3) (layers "F.Cu" "B.Cu") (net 9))
 (via (at 29.6386 -15.2827) (size 0.6) (drill 0.3) (layers "F.Cu" "B.Cu") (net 9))
 (via (at 35.7375 -17.1000) (size 0.6) (drill 0.3) (layers "F.Cu" "B.Cu") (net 9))
 (via (at 30.4375 -22.4000) (size 0.6) (drill 0.3) (layers "F.Cu" "B.Cu") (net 9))
 (via (at 21.2696 -14.3071) (size 0.6) (drill 0.3) (layers "F.Cu" "B.Cu") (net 9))
 (via (at 20.4750 -5.0000) (size 0.6) (drill 0.3) (layers "F.Cu" "B.Cu") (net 9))
 (via (at 34.4750 -5.0000) (size 0.6) (drill 0.3) (layers "F.Cu" "B.Cu") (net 9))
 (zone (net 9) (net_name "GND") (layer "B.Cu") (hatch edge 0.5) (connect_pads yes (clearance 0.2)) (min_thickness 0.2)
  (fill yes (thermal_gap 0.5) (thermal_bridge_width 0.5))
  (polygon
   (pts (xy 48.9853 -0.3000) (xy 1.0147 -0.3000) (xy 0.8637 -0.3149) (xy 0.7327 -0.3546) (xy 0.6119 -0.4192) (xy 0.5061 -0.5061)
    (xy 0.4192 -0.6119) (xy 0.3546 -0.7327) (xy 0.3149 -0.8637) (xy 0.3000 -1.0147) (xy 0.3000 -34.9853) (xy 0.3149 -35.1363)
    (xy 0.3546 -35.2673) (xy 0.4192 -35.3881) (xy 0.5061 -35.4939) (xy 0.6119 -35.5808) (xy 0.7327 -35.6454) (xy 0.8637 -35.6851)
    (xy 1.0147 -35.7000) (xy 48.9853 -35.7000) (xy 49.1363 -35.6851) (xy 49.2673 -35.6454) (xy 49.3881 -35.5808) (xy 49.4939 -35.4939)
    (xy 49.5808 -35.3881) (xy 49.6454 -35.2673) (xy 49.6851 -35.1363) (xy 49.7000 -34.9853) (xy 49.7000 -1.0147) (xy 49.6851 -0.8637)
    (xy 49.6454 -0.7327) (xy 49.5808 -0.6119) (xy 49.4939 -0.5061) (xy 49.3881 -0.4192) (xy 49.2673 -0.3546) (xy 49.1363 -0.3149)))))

